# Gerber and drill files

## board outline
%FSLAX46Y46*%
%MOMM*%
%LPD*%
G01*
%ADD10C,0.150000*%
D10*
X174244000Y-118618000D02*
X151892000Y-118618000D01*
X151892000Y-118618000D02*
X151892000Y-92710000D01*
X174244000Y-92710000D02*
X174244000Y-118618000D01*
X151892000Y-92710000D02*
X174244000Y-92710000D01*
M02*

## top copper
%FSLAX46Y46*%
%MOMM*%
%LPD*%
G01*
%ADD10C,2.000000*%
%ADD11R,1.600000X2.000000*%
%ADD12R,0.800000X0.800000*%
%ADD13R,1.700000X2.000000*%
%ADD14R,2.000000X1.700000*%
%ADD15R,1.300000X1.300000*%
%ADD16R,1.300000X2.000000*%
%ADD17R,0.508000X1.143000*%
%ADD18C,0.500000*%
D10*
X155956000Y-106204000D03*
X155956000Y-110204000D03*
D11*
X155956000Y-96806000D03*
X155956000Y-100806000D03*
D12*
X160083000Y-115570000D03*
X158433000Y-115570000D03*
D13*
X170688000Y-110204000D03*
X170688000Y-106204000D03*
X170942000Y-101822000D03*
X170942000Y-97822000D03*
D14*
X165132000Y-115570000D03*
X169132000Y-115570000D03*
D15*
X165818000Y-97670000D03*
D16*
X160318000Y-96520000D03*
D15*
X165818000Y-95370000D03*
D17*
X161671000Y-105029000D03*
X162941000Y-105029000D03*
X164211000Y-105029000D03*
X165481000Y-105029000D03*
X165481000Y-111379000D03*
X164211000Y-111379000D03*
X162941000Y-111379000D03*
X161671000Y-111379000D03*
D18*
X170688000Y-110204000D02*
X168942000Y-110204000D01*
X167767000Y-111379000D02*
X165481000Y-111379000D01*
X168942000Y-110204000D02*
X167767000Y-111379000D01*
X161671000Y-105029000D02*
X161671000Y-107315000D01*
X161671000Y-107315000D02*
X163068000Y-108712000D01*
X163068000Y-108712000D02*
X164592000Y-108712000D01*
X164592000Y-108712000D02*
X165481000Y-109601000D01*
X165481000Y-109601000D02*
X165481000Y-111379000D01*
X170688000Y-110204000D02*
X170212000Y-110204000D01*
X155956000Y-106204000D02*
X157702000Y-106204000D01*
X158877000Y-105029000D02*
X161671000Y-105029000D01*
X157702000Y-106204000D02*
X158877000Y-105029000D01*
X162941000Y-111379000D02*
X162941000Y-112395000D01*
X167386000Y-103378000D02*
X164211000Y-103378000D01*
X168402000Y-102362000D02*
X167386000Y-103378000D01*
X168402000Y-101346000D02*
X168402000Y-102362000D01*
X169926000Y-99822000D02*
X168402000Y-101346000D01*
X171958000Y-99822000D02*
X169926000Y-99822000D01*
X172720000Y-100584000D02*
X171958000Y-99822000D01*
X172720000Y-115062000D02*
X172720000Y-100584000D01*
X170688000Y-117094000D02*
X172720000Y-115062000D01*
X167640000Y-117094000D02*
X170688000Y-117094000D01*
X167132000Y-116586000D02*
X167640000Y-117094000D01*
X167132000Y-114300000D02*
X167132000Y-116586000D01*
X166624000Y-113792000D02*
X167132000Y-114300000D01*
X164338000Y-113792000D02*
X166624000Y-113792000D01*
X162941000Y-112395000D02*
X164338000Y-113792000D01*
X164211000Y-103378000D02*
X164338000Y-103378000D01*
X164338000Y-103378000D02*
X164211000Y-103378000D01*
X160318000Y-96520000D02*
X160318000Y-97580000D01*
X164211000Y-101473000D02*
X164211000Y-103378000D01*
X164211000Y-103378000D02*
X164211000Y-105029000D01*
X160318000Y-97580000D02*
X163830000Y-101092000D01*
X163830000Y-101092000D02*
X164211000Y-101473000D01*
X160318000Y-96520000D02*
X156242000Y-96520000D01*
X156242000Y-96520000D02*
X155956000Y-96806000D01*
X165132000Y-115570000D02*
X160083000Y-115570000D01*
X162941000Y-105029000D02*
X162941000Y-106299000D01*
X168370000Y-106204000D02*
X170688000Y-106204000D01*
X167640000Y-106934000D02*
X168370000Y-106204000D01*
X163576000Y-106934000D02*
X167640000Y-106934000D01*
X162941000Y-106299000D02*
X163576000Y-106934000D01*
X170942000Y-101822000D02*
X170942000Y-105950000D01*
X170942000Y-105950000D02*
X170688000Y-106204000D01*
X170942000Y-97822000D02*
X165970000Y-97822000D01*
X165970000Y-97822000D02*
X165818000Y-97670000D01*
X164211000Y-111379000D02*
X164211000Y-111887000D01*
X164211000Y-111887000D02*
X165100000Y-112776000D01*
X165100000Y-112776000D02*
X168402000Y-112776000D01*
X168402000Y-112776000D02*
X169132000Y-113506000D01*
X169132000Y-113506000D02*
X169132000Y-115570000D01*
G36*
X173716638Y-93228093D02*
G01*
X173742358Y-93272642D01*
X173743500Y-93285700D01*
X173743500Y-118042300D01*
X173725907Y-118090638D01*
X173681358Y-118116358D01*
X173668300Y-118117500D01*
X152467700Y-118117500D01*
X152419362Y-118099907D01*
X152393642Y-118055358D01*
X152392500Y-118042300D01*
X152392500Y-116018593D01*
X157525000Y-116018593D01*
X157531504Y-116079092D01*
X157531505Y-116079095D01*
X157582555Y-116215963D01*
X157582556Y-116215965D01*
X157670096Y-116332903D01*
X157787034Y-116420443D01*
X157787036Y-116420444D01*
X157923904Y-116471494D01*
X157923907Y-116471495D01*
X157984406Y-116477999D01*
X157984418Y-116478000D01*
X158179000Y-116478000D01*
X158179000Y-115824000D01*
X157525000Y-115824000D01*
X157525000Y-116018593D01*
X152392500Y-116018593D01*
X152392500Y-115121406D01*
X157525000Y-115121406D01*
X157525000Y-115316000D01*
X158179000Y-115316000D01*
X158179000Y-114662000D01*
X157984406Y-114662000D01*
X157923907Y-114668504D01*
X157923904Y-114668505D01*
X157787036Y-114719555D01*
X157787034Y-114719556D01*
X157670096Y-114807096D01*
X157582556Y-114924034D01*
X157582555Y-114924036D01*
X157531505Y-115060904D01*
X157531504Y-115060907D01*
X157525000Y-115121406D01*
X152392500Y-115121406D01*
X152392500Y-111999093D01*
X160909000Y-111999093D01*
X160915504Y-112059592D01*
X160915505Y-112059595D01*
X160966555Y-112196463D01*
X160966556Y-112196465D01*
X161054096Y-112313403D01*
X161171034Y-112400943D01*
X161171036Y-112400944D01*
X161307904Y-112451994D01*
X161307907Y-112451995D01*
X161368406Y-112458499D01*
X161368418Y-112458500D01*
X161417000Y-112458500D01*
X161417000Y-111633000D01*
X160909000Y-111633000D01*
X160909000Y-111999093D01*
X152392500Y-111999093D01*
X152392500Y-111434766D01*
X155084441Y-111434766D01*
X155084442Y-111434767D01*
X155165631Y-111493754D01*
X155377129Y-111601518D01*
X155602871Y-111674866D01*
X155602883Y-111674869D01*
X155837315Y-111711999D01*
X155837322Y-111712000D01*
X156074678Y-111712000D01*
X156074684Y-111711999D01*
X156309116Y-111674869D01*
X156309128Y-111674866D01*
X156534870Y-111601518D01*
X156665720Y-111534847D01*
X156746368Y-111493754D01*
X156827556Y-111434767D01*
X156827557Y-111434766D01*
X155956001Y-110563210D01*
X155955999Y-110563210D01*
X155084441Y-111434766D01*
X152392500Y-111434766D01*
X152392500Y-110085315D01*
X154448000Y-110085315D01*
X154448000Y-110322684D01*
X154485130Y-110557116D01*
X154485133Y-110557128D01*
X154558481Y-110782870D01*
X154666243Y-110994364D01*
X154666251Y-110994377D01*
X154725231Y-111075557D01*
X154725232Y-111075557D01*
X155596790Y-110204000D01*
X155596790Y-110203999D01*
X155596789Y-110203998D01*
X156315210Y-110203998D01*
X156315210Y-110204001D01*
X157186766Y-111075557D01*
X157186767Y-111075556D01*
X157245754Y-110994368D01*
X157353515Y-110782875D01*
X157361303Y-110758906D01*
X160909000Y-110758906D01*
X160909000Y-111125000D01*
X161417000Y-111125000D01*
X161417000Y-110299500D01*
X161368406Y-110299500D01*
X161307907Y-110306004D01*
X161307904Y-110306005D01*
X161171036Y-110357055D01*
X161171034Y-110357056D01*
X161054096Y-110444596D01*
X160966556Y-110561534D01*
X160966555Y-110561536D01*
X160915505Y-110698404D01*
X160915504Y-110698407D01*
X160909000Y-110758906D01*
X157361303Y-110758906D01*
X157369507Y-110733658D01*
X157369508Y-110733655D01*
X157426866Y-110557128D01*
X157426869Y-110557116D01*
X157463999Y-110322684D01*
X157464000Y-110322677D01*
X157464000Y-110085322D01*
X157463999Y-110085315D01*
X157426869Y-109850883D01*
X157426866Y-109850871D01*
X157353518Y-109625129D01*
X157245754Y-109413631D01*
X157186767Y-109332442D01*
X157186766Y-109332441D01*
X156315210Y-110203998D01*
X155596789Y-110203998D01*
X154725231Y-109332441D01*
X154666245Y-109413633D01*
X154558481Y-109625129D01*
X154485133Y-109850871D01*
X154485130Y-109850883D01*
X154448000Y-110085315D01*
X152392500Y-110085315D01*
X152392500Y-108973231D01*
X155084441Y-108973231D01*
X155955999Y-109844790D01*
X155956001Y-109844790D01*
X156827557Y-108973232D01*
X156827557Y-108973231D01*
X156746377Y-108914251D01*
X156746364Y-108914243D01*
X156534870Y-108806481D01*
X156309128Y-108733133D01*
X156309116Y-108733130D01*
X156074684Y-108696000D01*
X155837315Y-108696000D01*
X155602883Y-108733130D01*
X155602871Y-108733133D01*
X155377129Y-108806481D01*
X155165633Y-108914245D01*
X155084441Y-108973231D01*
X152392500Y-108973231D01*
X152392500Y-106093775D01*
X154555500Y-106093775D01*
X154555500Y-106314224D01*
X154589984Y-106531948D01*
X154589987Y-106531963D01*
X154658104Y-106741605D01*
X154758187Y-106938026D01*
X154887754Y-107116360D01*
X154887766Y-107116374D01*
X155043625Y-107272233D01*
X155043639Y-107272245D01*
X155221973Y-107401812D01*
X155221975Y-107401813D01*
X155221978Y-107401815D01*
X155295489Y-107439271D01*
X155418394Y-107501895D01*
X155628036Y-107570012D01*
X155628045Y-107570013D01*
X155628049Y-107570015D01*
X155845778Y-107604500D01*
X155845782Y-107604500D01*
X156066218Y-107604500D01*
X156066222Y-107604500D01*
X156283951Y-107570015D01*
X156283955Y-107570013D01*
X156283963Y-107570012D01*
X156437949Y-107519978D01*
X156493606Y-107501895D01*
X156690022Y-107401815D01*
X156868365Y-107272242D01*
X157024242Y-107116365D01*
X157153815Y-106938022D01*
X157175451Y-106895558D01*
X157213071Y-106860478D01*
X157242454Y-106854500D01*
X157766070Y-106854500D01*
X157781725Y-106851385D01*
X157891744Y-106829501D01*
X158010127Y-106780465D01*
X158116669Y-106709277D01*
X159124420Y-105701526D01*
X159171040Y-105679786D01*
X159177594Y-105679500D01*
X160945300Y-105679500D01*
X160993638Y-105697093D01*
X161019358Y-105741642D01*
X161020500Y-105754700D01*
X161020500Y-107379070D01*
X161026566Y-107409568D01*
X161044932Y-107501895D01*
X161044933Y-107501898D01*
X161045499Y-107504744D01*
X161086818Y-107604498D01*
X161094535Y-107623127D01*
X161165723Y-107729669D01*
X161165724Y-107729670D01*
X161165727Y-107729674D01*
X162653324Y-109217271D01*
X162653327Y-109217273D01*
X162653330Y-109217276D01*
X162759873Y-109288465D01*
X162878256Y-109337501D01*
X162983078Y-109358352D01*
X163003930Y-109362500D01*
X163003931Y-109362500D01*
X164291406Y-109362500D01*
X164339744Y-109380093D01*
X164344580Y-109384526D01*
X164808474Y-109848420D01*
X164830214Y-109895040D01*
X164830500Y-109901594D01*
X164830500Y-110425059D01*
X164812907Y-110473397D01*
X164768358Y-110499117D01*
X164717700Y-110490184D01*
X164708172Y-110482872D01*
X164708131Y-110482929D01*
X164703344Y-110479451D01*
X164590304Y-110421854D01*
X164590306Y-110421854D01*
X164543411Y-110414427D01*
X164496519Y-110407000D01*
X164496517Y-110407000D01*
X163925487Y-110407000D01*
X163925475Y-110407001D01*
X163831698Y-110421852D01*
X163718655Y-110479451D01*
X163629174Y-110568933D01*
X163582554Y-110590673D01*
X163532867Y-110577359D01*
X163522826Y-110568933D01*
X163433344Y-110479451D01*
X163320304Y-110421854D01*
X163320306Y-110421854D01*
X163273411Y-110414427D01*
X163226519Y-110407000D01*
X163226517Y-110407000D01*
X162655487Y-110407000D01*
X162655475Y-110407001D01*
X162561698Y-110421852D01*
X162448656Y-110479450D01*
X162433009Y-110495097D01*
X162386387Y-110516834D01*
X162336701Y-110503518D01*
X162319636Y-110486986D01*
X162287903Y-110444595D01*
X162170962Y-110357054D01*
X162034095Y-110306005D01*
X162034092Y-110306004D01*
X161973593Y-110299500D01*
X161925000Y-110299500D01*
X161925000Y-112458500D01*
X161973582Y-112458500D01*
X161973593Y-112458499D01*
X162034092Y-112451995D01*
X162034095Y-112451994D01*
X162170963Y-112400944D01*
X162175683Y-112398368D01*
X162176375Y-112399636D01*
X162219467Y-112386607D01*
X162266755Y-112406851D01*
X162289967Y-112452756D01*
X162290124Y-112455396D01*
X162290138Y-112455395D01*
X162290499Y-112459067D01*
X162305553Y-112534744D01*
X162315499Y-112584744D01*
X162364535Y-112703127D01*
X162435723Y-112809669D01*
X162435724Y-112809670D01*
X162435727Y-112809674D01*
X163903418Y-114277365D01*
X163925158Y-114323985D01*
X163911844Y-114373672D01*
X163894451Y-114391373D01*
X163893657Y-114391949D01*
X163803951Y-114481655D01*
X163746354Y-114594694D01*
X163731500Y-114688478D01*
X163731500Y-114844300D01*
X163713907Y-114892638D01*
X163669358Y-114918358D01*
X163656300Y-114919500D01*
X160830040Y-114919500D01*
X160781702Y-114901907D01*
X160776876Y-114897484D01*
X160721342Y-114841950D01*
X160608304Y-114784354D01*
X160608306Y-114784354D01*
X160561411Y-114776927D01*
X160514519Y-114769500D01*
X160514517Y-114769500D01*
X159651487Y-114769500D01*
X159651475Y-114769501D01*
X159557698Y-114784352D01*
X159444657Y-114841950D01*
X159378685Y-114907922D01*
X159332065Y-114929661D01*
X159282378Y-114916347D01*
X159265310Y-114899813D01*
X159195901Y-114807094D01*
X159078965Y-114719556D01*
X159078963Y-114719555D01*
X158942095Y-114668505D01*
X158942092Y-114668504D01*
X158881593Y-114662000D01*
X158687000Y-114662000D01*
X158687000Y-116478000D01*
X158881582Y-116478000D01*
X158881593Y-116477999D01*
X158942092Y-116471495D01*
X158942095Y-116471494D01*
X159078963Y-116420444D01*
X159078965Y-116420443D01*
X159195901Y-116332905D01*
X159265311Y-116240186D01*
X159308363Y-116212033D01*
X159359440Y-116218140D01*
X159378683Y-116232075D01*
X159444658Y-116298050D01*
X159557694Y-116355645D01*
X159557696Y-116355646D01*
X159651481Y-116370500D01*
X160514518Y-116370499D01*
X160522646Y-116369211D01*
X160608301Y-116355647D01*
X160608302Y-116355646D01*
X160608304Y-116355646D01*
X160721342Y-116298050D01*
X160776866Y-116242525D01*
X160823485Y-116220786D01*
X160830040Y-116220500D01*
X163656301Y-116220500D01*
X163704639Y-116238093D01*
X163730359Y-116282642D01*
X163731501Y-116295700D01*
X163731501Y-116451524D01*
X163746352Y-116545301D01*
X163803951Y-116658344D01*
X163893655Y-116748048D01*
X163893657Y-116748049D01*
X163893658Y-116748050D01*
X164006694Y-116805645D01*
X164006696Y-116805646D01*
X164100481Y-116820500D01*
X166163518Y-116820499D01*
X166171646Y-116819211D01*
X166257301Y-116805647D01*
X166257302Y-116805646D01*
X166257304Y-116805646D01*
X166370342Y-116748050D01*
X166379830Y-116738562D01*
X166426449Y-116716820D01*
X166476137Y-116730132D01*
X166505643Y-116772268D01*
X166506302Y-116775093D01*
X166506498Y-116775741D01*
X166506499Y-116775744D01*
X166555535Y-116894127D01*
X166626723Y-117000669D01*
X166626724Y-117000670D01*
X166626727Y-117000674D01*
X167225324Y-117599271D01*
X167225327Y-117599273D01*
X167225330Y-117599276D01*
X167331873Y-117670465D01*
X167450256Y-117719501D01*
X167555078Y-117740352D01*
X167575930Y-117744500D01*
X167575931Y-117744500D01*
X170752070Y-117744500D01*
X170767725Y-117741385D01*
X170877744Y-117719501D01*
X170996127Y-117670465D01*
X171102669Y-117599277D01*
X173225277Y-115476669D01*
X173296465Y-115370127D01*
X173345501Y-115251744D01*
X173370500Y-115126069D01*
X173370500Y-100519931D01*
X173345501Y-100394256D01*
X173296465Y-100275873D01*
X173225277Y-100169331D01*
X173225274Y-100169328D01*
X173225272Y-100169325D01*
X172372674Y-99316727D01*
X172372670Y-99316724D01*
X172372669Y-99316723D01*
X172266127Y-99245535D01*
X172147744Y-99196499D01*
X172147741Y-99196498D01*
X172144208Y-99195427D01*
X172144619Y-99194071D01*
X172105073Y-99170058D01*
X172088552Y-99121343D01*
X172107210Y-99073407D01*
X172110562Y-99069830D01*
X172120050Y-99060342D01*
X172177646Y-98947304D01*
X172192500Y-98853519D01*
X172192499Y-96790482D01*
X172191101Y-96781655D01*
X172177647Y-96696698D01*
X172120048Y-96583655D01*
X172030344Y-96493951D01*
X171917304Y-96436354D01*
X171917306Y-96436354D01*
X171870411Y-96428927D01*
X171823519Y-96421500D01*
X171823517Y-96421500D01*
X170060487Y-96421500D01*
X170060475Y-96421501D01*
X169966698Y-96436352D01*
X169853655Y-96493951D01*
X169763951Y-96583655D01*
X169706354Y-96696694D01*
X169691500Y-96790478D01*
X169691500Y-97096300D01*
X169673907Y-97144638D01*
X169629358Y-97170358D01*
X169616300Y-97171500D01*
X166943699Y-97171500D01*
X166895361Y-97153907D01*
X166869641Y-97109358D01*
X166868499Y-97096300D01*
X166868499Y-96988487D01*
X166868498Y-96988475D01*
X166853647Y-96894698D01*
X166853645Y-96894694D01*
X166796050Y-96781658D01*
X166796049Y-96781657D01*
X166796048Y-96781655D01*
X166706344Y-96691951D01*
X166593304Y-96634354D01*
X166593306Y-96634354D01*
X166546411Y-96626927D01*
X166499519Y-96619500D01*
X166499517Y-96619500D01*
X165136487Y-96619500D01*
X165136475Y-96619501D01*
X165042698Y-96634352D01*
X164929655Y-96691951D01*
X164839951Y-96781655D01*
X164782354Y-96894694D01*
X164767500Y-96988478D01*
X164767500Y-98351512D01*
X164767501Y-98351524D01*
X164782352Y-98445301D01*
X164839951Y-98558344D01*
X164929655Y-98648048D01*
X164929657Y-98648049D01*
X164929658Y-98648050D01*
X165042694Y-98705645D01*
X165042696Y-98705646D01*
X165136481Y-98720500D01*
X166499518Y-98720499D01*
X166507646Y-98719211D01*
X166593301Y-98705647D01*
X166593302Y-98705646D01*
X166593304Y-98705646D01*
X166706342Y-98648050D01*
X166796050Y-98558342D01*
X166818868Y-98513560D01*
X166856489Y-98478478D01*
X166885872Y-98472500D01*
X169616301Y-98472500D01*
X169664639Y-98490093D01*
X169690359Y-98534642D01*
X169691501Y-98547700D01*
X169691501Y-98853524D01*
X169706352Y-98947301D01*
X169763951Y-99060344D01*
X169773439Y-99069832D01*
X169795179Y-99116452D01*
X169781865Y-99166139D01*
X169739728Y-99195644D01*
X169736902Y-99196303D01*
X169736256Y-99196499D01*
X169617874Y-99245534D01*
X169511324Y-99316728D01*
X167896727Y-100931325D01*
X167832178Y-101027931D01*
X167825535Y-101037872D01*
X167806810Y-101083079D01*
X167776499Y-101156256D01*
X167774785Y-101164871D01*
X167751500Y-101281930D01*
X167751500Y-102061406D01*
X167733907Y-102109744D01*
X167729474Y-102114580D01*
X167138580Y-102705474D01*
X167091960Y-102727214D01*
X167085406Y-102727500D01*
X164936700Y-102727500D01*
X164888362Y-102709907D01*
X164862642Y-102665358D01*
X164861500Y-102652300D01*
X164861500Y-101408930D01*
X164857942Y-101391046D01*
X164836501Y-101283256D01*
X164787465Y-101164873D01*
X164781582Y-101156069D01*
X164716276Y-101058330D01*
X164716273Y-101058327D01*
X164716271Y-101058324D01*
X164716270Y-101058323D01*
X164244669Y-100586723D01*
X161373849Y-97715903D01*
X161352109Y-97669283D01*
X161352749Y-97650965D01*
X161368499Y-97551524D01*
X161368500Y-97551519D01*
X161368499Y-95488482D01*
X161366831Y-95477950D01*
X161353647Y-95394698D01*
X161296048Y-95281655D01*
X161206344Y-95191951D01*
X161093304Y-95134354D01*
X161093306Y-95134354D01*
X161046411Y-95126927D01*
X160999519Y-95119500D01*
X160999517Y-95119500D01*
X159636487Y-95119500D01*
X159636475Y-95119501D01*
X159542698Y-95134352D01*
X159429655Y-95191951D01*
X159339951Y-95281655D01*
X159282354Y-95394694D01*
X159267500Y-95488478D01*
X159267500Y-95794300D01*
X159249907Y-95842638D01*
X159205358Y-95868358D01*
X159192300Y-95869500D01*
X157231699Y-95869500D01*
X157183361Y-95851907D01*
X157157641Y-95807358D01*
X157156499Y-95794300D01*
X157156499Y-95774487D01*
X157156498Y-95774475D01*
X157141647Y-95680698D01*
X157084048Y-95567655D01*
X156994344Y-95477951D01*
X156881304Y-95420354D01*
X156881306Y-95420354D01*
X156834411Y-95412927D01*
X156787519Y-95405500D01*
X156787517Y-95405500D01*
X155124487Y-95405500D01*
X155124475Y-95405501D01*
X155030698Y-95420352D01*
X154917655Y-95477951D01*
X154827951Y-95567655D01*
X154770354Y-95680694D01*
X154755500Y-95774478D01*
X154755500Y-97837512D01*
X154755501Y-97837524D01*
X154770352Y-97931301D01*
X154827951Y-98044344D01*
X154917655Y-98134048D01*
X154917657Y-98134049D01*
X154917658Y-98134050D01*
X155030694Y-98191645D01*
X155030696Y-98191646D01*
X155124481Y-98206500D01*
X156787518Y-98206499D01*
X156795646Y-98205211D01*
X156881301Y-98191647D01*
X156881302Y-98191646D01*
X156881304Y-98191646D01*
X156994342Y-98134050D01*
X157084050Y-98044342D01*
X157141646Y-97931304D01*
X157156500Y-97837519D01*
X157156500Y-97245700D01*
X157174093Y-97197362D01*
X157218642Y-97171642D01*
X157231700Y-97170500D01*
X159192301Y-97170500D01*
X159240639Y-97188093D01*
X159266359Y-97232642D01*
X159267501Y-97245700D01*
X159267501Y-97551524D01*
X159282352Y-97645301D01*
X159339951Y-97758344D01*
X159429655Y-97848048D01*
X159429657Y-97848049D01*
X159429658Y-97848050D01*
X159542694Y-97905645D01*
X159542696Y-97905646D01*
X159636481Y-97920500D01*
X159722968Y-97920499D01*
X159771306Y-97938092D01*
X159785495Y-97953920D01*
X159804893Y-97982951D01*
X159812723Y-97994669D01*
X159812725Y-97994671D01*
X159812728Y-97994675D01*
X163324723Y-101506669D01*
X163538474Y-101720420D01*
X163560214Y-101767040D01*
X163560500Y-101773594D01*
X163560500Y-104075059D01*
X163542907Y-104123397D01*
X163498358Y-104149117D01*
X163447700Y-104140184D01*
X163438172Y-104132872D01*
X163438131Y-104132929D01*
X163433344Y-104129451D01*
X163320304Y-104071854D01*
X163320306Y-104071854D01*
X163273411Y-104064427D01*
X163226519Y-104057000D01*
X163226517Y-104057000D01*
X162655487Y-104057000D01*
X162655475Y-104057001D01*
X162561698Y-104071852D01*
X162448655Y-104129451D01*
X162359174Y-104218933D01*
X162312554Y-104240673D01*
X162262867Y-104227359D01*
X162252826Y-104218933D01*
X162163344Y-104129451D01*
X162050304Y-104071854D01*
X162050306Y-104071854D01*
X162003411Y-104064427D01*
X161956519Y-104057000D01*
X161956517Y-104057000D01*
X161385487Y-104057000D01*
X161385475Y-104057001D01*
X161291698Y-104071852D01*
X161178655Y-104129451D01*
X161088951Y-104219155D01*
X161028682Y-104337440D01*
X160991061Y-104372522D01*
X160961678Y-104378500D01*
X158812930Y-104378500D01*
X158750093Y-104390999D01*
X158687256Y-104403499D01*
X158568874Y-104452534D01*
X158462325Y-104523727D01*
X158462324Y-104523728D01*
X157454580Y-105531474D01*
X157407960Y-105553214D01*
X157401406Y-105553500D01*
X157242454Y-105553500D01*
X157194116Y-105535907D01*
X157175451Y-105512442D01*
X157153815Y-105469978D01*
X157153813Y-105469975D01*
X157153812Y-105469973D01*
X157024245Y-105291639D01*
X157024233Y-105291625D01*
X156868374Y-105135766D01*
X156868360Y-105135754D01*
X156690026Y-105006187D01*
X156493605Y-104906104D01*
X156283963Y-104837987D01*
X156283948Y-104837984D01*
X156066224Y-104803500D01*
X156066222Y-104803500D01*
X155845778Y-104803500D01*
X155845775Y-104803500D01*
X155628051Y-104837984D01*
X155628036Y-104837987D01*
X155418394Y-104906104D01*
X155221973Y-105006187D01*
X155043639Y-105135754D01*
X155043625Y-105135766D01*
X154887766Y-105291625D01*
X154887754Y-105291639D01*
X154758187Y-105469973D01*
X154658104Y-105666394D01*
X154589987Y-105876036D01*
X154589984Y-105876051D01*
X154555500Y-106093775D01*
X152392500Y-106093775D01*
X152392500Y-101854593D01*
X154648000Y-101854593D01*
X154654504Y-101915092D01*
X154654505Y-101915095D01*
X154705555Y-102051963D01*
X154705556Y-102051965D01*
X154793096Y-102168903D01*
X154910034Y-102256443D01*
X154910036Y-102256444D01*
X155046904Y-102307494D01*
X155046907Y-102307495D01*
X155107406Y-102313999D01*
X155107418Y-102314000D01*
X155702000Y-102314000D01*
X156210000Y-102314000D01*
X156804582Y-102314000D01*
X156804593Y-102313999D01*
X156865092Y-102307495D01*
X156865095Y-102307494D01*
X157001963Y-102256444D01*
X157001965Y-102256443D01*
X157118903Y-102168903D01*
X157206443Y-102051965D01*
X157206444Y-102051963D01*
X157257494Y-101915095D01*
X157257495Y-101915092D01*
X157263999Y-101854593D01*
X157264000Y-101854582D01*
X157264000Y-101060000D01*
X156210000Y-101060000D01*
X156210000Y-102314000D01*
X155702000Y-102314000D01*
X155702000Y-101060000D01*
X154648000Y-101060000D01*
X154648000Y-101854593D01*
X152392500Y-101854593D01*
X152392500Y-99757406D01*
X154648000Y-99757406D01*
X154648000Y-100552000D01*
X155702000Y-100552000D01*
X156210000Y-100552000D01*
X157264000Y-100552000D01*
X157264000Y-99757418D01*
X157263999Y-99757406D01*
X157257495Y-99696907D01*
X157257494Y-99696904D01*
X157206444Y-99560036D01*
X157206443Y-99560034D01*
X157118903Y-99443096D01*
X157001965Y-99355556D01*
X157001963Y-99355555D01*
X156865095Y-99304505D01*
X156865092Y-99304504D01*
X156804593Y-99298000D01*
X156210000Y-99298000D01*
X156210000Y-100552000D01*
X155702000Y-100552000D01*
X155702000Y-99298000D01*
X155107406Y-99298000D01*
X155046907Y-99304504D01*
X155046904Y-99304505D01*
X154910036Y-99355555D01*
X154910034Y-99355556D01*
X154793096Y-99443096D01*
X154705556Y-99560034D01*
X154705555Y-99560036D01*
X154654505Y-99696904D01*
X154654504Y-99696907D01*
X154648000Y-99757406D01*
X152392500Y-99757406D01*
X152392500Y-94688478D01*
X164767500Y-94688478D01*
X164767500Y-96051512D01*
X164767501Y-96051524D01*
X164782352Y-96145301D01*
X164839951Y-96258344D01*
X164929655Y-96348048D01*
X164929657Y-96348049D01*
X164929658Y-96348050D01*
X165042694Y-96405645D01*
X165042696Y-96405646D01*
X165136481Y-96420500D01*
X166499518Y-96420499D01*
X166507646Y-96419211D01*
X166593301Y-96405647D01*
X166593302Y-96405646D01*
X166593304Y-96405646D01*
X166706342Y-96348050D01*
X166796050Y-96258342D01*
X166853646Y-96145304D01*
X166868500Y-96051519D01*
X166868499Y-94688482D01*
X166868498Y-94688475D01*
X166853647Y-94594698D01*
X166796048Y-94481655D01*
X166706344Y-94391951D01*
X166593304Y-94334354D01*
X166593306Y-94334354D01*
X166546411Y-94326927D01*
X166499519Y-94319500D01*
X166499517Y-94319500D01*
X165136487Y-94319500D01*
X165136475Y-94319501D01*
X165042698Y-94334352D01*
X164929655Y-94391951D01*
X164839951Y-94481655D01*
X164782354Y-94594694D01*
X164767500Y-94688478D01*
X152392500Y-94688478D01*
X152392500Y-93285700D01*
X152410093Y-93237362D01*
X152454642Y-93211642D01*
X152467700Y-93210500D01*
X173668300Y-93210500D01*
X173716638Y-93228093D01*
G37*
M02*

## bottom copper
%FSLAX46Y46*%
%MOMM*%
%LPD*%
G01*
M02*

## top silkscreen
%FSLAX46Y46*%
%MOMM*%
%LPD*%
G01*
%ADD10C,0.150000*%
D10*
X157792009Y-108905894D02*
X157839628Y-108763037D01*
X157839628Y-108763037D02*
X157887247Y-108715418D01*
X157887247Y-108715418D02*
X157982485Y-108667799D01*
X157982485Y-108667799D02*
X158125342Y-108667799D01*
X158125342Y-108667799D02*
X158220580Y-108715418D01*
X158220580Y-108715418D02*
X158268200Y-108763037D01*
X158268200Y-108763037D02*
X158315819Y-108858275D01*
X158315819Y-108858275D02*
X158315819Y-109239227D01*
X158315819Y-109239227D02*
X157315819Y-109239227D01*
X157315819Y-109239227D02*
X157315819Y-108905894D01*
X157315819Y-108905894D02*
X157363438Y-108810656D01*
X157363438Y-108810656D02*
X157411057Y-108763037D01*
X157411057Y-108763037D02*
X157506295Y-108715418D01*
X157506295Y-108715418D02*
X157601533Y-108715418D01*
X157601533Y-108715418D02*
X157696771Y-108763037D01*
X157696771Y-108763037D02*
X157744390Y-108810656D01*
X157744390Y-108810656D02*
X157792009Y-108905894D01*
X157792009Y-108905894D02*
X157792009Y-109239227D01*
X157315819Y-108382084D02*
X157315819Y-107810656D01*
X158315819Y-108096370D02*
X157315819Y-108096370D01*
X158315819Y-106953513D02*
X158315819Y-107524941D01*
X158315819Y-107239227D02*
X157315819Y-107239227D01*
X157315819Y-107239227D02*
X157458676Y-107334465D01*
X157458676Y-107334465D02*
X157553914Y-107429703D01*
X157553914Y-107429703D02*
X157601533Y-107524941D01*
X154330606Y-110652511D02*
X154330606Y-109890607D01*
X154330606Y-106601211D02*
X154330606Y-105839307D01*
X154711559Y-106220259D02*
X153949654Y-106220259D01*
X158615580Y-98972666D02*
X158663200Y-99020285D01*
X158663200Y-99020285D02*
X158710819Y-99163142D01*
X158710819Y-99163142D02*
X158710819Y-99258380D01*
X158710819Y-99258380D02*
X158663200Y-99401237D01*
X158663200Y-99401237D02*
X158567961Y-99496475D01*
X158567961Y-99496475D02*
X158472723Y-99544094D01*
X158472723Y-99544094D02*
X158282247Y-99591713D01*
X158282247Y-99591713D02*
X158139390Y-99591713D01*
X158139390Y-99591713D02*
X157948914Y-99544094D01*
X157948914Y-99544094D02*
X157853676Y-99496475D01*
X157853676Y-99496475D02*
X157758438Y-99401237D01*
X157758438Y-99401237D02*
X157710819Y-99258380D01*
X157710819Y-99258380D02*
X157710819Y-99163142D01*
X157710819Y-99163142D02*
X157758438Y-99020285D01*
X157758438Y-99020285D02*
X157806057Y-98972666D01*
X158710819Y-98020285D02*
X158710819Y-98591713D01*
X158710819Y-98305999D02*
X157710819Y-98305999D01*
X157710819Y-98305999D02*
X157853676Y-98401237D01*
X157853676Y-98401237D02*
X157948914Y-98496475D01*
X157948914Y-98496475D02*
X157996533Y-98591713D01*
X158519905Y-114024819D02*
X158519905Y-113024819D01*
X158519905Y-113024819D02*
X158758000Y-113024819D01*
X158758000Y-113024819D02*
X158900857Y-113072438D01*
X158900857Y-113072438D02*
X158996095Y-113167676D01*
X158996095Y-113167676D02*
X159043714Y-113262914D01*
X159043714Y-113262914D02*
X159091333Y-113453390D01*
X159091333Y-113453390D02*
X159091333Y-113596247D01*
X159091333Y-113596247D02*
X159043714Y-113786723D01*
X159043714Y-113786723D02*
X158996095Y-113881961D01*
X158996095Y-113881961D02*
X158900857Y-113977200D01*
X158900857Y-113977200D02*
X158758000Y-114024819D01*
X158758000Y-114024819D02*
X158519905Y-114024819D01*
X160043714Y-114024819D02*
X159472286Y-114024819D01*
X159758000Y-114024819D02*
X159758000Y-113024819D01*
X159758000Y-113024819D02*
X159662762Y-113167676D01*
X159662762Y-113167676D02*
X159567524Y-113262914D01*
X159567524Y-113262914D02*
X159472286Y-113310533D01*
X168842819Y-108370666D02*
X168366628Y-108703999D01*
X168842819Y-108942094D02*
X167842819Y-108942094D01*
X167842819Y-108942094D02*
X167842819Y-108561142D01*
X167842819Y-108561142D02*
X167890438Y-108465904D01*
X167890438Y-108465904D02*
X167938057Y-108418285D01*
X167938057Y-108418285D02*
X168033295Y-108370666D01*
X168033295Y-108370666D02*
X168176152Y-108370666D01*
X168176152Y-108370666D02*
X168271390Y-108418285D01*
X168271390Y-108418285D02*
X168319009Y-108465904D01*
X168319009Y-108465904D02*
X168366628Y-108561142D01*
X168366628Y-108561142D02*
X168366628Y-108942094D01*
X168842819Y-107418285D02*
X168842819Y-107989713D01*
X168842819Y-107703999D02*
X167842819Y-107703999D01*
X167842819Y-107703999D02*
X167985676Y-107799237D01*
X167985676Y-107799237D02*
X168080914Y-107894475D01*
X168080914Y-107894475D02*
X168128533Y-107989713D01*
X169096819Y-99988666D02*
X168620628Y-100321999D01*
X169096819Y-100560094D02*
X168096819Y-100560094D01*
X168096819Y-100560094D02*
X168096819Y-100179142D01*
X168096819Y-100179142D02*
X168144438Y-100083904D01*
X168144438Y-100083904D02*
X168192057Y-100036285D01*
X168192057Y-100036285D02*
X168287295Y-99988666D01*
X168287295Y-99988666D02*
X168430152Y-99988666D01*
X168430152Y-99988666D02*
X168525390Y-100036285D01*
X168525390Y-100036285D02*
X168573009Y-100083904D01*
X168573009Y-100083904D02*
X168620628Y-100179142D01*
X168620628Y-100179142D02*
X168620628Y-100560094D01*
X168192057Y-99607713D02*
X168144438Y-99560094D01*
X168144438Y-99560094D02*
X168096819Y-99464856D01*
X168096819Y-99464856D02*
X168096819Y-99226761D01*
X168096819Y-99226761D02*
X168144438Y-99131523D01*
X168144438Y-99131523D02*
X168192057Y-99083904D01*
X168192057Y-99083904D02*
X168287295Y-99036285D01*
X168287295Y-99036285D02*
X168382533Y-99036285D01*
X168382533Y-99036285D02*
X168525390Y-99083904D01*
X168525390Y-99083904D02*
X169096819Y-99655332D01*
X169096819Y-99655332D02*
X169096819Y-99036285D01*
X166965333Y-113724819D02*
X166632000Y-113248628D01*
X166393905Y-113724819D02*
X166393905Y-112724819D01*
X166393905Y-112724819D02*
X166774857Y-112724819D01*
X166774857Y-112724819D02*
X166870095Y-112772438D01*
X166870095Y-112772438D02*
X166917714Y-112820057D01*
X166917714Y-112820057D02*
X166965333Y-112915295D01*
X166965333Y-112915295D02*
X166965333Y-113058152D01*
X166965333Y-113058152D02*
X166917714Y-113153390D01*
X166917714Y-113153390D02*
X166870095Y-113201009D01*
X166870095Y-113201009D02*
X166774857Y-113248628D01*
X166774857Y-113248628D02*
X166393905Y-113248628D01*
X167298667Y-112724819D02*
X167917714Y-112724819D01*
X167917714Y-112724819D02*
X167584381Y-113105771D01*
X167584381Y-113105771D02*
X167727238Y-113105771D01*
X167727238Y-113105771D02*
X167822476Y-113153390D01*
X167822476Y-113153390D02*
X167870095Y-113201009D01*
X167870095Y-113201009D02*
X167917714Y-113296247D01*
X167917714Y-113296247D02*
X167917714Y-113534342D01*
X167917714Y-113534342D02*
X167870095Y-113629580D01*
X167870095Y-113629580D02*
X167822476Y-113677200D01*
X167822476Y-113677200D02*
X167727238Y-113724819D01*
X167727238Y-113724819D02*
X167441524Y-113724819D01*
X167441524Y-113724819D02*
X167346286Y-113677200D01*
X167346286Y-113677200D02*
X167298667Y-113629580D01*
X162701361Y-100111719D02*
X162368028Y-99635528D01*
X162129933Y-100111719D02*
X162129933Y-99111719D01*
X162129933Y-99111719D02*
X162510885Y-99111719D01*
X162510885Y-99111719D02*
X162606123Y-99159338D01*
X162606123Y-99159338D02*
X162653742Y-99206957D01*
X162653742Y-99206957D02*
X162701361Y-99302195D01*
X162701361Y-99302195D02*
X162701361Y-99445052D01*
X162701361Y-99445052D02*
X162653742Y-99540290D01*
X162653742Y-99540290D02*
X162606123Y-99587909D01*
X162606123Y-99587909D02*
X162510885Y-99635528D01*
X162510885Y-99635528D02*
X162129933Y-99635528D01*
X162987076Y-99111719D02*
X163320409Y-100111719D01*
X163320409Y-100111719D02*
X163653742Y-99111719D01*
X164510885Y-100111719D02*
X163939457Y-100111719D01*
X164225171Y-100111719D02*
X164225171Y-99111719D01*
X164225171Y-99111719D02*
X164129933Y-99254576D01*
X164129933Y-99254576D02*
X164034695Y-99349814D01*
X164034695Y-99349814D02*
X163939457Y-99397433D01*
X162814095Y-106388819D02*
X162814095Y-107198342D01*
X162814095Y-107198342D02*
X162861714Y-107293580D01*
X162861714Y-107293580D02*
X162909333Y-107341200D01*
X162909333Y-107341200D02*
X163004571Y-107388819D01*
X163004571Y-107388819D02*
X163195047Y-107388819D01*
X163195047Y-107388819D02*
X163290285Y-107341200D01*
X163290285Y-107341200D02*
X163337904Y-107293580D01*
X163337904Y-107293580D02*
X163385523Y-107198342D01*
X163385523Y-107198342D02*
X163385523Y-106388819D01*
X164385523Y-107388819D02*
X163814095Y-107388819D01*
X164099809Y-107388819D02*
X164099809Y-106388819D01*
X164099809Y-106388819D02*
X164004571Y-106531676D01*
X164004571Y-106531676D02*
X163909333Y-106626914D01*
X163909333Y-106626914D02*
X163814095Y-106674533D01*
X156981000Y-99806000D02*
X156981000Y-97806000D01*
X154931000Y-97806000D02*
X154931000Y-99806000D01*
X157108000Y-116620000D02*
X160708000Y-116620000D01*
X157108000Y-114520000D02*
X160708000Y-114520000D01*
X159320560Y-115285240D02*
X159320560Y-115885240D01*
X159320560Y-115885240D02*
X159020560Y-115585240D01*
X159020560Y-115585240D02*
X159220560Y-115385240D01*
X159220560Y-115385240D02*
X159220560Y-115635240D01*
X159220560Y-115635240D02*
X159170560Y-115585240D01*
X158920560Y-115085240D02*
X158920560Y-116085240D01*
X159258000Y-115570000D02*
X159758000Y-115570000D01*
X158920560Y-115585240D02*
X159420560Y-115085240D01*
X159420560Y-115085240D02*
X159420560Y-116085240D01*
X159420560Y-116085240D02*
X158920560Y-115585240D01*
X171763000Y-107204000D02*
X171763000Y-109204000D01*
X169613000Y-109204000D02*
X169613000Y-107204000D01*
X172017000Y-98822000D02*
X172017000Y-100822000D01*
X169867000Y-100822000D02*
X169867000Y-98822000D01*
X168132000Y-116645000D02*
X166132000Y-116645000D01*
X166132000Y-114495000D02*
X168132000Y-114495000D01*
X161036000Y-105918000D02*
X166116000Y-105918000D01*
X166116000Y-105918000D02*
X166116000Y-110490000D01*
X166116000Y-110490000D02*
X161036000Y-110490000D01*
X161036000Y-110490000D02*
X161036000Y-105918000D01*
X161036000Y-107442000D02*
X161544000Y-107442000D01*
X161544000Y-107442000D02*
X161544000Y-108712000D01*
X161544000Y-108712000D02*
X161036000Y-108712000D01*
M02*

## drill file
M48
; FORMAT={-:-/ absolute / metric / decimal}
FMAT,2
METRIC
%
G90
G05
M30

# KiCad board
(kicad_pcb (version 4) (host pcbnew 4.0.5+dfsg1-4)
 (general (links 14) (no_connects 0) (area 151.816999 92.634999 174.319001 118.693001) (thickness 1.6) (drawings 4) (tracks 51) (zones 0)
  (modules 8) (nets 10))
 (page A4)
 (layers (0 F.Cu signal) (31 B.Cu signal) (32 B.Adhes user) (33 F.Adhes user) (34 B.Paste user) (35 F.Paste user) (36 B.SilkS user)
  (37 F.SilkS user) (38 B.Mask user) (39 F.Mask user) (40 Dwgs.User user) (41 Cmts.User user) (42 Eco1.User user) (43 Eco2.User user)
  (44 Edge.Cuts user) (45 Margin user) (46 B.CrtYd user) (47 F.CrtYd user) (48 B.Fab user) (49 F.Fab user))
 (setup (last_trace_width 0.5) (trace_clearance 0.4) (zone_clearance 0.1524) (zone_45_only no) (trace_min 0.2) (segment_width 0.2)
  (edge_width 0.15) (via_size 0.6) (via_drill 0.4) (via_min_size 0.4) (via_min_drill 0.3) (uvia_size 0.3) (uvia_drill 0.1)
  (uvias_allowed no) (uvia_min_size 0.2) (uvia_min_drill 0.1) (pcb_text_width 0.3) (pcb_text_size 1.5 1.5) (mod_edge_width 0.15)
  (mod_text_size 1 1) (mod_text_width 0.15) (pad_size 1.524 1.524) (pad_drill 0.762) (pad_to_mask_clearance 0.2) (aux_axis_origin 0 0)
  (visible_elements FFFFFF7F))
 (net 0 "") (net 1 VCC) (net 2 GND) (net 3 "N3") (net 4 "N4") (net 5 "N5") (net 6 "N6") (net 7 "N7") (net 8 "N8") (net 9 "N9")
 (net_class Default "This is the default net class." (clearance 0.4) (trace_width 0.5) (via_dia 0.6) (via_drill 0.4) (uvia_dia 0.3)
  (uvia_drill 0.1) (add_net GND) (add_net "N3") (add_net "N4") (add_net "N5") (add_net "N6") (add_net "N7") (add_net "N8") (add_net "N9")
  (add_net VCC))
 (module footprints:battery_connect (layer F.Cu) (at 155.956 108.204 270)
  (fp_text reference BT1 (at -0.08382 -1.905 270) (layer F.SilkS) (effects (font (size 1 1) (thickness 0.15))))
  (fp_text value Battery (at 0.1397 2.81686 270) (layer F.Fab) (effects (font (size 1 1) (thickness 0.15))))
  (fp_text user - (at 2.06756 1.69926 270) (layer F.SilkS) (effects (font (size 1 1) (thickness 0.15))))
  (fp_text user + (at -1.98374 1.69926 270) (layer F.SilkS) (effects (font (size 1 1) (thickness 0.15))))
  (pad 1 smd circle (at -2 0 270) (size 2 2) (layers F.Cu F.Paste F.Mask) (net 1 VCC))
  (pad 2 smd circle (at 2 0 270) (size 2 2) (layers F.Cu F.Paste F.Mask) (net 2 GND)))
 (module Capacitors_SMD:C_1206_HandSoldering (layer F.Cu) (at 155.956 98.806 270)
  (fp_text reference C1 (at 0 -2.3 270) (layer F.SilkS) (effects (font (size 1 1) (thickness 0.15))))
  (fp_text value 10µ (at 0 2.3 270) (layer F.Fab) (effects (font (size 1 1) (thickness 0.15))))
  (fp_line (start 1 -1.025) (end -1 -1.025) (layer F.SilkS) (width 0.15))
  (fp_line (start -1 1.025) (end 1 1.025) (layer F.SilkS) (width 0.15))
  (pad 1 smd rect (at -2 0 270) (size 2 1.6) (layers F.Cu F.Paste F.Mask) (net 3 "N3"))
  (pad 2 smd rect (at 2 0 270) (size 2 1.6) (layers F.Cu F.Paste F.Mask) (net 2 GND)))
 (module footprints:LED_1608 (layer F.Cu) (at 159.258 115.57)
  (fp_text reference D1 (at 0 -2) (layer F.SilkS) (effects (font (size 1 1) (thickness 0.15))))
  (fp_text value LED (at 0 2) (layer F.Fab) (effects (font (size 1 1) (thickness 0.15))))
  (fp_line (start -2.15 1.05) (end 1.45 1.05) (layer F.SilkS) (width 0.15))
  (fp_line (start -2.15 -1.05) (end 1.45 -1.05) (layer F.SilkS) (width 0.15))
  (fp_line (start 0.06256 -0.28476) (end 0.06256 0.31524) (layer F.SilkS) (width 0.15))
  (fp_line (start 0.06256 0.31524) (end -0.23744 0.01524) (layer F.SilkS) (width 0.15))
  (fp_line (start -0.23744 0.01524) (end -0.03744 -0.18476) (layer F.SilkS) (width 0.15))
  (fp_line (start -0.03744 -0.18476) (end -0.03744 0.06524) (layer F.SilkS) (width 0.15))
  (fp_line (start -0.03744 0.06524) (end -0.08744 0.01524) (layer F.SilkS) (width 0.15))
  (fp_line (start -0.33744 -0.48476) (end -0.33744 0.51524) (layer F.SilkS) (width 0.15))
  (fp_line (start 0 0) (end 0.5 0) (layer F.SilkS) (width 0.15))
  (fp_line (start -0.33744 0.01524) (end 0.16256 -0.48476) (layer F.SilkS) (width 0.15))
  (fp_line (start 0.16256 -0.48476) (end 0.16256 0.51524) (layer F.SilkS) (width 0.15))
  (fp_line (start 0.16256 0.51524) (end -0.33744 0.01524) (layer F.SilkS) (width 0.15))
  (pad 2 smd rect (at 0.825 0 180) (size 0.8 0.8) (layers F.Cu F.Paste F.Mask) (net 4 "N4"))
  (pad 1 smd rect (at -0.825 0 180) (size 0.8 0.8) (layers F.Cu F.Paste F.Mask) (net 2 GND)))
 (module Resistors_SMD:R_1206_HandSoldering (layer F.Cu) (at 170.688 108.204 90)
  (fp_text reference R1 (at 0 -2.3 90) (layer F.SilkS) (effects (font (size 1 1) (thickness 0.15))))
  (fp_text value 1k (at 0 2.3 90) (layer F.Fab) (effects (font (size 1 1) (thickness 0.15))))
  (fp_line (start 1 1.075) (end -1 1.075) (layer F.SilkS) (width 0.15))
  (fp_line (start -1 -1.075) (end 1 -1.075) (layer F.SilkS) (width 0.15))
  (pad 1 smd rect (at -2 0 90) (size 2 1.7) (layers F.Cu F.Paste F.Mask) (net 1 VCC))
  (pad 2 smd rect (at 2 0 90) (size 2 1.7) (layers F.Cu F.Paste F.Mask) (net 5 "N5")))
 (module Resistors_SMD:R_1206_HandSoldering (layer F.Cu) (at 170.942 99.822 90)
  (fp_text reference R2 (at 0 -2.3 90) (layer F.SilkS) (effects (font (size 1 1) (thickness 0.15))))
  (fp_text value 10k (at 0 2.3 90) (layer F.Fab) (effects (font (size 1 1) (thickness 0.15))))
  (fp_line (start 1 1.075) (end -1 1.075) (layer F.SilkS) (width 0.15))
  (fp_line (start -1 -1.075) (end 1 -1.075) (layer F.SilkS) (width 0.15))
  (pad 1 smd rect (at -2 0 90) (size 2 1.7) (layers F.Cu F.Paste F.Mask) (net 5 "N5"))
  (pad 2 smd rect (at 2 0 90) (size 2 1.7) (layers F.Cu F.Paste F.Mask) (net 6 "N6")))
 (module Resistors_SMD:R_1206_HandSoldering (layer F.Cu) (at 167.132 115.57)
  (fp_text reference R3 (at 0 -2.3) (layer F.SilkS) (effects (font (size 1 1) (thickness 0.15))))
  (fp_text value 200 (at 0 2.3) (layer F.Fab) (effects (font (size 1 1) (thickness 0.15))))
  (fp_line (start 1 1.075) (end -1 1.075) (layer F.SilkS) (width 0.15))
  (fp_line (start -1 -1.075) (end 1 -1.075) (layer F.SilkS) (width 0.15))
  (pad 1 smd rect (at -2 0) (size 2 1.7) (layers F.Cu F.Paste F.Mask) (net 4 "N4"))
  (pad 2 smd rect (at 2 0) (size 2 1.7) (layers F.Cu F.Paste F.Mask) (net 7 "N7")))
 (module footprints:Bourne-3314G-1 (layer F.Cu) (at 163.068 96.52 270)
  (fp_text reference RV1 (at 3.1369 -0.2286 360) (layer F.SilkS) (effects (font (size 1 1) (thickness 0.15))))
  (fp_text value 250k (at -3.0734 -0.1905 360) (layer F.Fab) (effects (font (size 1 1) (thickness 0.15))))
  (pad 1 smd rect (at 1.15 -2.75 270) (size 1.3 1.3) (layers F.Cu F.Paste F.Mask) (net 6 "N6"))
  (pad 2 smd rect (at 0 2.75 270) (size 2 1.3) (layers F.Cu F.Paste F.Mask) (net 3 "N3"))
  (pad 3 smd rect (at -1.15 -2.75 270) (size 1.3 1.3) (layers F.Cu F.Paste F.Mask) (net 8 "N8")))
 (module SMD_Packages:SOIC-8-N (layer F.Cu) (at 163.576 108.204)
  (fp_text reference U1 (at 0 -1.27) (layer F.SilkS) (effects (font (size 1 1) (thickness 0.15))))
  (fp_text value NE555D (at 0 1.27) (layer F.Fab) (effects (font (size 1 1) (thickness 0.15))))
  (fp_line (start -2.54 -2.286) (end 2.54 -2.286) (layer F.SilkS) (width 0.15))
  (fp_line (start 2.54 -2.286) (end 2.54 2.286) (layer F.SilkS) (width 0.15))
  (fp_line (start 2.54 2.286) (end -2.54 2.286) (layer F.SilkS) (width 0.15))
  (fp_line (start -2.54 2.286) (end -2.54 -2.286) (layer F.SilkS) (width 0.15))
  (fp_line (start -2.54 -0.762) (end -2.032 -0.762) (layer F.SilkS) (width 0.15))
  (fp_line (start -2.032 -0.762) (end -2.032 0.508) (layer F.SilkS) (width 0.15))
  (fp_line (start -2.032 0.508) (end -2.54 0.508) (layer F.SilkS) (width 0.15))
  (pad 8 smd rect (at -1.905 -3.175) (size 0.508 1.143) (layers F.Cu F.Paste F.Mask) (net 1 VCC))
  (pad 7 smd rect (at -0.635 -3.175) (size 0.508 1.143) (layers F.Cu F.Paste F.Mask) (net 5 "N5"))
  (pad 6 smd rect (at 0.635 -3.175) (size 0.508 1.143) (layers F.Cu F.Paste F.Mask) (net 3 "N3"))
  (pad 5 smd rect (at 1.905 -3.175) (size 0.508 1.143) (layers F.Cu F.Paste F.Mask) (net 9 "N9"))
  (pad 4 smd rect (at 1.905 3.175) (size 0.508 1.143) (layers F.Cu F.Paste F.Mask) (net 1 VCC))
  (pad 3 smd rect (at 0.635 3.175) (size 0.508 1.143) (layers F.Cu F.Paste F.Mask) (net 7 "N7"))
  (pad 2 smd rect (at -0.635 3.175) (size 0.508 1.143) (layers F.Cu F.Paste F.Mask) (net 3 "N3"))
  (pad 1 smd rect (at -1.905 3.175) (size 0.508 1.143) (layers F.Cu F.Paste F.Mask) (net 2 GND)))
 (gr_line (start 174.244 118.618) (end 151.892 118.618) (angle 90) (layer Edge.Cuts) (width 0.15))
 (gr_line (start 151.892 118.618) (end 151.892 92.71) (angle 90) (layer Edge.Cuts) (width 0.15))
 (gr_line (start 174.244 92.71) (end 174.244 118.618) (angle 90) (layer Edge.Cuts) (width 0.15))
 (gr_line (start 151.892 92.71) (end 174.244 92.71) (angle 90) (layer Edge.Cuts) (width 0.15))
 (segment (start 170.688 110.204) (end 168.942 110.204) (width 0.5) (layer F.Cu) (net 1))
 (segment (start 167.767 111.379) (end 165.481 111.379) (width 0.5) (layer F.Cu) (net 1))
 (segment (start 168.942 110.204) (end 167.767 111.379) (width 0.5) (layer F.Cu) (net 1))
 (segment (start 161.671 105.029) (end 161.671 107.315) (width 0.5) (layer F.Cu) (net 1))
 (segment (start 161.671 107.315) (end 163.068 108.712) (width 0.5) (layer F.Cu) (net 1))
 (segment (start 163.068 108.712) (end 164.592 108.712) (width 0.5) (layer F.Cu) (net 1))
 (segment (start 164.592 108.712) (end 165.481 109.601) (width 0.5) (layer F.Cu) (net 1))
 (segment (start 165.481 109.601) (end 165.481 111.379) (width 0.5) (layer F.Cu) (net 1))
 (segment (start 170.688 110.204) (end 170.212 110.204) (width 0.5) (layer F.Cu) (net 1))
 (segment (start 155.956 106.204) (end 157.702 106.204) (width 0.5) (layer F.Cu) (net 1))
 (segment (start 158.877 105.029) (end 161.671 105.029) (width 0.5) (layer F.Cu) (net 1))
 (segment (start 157.702 106.204) (end 158.877 105.029) (width 0.5) (layer F.Cu) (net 1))
 (segment (start 162.941 111.379) (end 162.941 112.395) (width 0.5) (layer F.Cu) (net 3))
 (segment (start 167.386 103.378) (end 164.211 103.378) (width 0.5) (layer F.Cu) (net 3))
 (segment (start 168.402 102.362) (end 167.386 103.378) (width 0.5) (layer F.Cu) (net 3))
 (segment (start 168.402 101.346) (end 168.402 102.362) (width 0.5) (layer F.Cu) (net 3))
 (segment (start 169.926 99.822) (end 168.402 101.346) (width 0.5) (layer F.Cu) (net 3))
 (segment (start 171.958 99.822) (end 169.926 99.822) (width 0.5) (layer F.Cu) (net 3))
 (segment (start 172.72 100.584) (end 171.958 99.822) (width 0.5) (layer F.Cu) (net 3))
 (segment (start 172.72 115.062) (end 172.72 100.584) (width 0.5) (layer F.Cu) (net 3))
 (segment (start 170.688 117.094) (end 172.72 115.062) (width 0.5) (layer F.Cu) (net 3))
 (segment (start 167.64 117.094) (end 170.688 117.094) (width 0.5) (layer F.Cu) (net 3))
 (segment (start 167.132 116.586) (end 167.64 117.094) (width 0.5) (layer F.Cu) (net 3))
 (segment (start 167.132 114.3) (end 167.132 116.586) (width 0.5) (layer F.Cu) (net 3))
 (segment (start 166.624 113.792) (end 167.132 114.3) (width 0.5) (layer F.Cu) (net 3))
 (segment (start 164.338 113.792) (end 166.624 113.792) (width 0.5) (layer F.Cu) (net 3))
 (segment (start 162.941 112.395) (end 164.338 113.792) (width 0.5) (layer F.Cu) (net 3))
 (segment (start 164.211 103.378) (end 164.338 103.378) (width 0.5) (layer F.Cu) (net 3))
 (segment (start 164.338 103.378) (end 164.211 103.378) (width 0.5) (layer F.Cu) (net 3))
 (segment (start 160.318 96.52) (end 160.318 97.58) (width 0.5) (layer F.Cu) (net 3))
 (segment (start 164.211 101.473) (end 164.211 103.378) (width 0.5) (layer F.Cu) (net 3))
 (segment (start 164.211 103.378) (end 164.211 105.029) (width 0.5) (layer F.Cu) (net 3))
 (segment (start 160.318 97.58) (end 163.83 101.092) (width 0.5) (layer F.Cu) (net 3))
 (segment (start 163.83 101.092) (end 164.211 101.473) (width 0.5) (layer F.Cu) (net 3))
 (segment (start 160.318 96.52) (end 156.242 96.52) (width 0.5) (layer F.Cu) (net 3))
 (segment (start 156.242 96.52) (end 155.956 96.806) (width 0.5) (layer F.Cu) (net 3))
 (segment (start 165.132 115.57) (end 160.083 115.57) (width 0.5) (layer F.Cu) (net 4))
 (segment (start 162.941 105.029) (end 162.941 106.299) (width 0.5) (layer F.Cu) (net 5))
 (segment (start 168.37 106.204) (end 170.688 106.204) (width 0.5) (layer F.Cu) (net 5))
 (segment (start 167.64 106.934) (end 168.37 106.204) (width 0.5) (layer F.Cu) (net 5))
 (segment (start 163.576 106.934) (end 167.64 106.934) (width 0.5) (layer F.Cu) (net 5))
 (segment (start 162.941 106.299) (end 163.576 106.934) (width 0.5) (layer F.Cu) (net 5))
 (segment (start 170.942 101.822) (end 170.942 105.95) (width 0.5) (layer F.Cu) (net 5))
 (segment (start 170.942 105.95) (end 170.688 106.204) (width 0.5) (layer F.Cu) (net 5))
 (segment (start 170.942 97.822) (end 165.97 97.822) (width 0.5) (layer F.Cu) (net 6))
 (segment (start 165.97 97.822) (end 165.818 97.67) (width 0.5) (layer F.Cu) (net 6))
 (segment (start 164.211 111.379) (end 164.211 111.887) (width 0.5) (layer F.Cu) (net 7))
 (segment (start 164.211 111.887) (end 165.1 112.776) (width 0.5) (layer F.Cu) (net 7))
 (segment (start 165.1 112.776) (end 168.402 112.776) (width 0.5) (layer F.Cu) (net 7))
 (segment (start 168.402 112.776) (end 169.132 113.506) (width 0.5) (layer F.Cu) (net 7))
 (segment (start 169.132 113.506) (end 169.132 115.57) (width 0.5) (layer F.Cu) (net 7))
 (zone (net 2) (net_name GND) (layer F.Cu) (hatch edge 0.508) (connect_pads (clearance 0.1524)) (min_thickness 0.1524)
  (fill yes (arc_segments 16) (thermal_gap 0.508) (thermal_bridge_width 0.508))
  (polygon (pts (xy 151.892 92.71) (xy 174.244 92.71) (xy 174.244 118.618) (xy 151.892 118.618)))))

